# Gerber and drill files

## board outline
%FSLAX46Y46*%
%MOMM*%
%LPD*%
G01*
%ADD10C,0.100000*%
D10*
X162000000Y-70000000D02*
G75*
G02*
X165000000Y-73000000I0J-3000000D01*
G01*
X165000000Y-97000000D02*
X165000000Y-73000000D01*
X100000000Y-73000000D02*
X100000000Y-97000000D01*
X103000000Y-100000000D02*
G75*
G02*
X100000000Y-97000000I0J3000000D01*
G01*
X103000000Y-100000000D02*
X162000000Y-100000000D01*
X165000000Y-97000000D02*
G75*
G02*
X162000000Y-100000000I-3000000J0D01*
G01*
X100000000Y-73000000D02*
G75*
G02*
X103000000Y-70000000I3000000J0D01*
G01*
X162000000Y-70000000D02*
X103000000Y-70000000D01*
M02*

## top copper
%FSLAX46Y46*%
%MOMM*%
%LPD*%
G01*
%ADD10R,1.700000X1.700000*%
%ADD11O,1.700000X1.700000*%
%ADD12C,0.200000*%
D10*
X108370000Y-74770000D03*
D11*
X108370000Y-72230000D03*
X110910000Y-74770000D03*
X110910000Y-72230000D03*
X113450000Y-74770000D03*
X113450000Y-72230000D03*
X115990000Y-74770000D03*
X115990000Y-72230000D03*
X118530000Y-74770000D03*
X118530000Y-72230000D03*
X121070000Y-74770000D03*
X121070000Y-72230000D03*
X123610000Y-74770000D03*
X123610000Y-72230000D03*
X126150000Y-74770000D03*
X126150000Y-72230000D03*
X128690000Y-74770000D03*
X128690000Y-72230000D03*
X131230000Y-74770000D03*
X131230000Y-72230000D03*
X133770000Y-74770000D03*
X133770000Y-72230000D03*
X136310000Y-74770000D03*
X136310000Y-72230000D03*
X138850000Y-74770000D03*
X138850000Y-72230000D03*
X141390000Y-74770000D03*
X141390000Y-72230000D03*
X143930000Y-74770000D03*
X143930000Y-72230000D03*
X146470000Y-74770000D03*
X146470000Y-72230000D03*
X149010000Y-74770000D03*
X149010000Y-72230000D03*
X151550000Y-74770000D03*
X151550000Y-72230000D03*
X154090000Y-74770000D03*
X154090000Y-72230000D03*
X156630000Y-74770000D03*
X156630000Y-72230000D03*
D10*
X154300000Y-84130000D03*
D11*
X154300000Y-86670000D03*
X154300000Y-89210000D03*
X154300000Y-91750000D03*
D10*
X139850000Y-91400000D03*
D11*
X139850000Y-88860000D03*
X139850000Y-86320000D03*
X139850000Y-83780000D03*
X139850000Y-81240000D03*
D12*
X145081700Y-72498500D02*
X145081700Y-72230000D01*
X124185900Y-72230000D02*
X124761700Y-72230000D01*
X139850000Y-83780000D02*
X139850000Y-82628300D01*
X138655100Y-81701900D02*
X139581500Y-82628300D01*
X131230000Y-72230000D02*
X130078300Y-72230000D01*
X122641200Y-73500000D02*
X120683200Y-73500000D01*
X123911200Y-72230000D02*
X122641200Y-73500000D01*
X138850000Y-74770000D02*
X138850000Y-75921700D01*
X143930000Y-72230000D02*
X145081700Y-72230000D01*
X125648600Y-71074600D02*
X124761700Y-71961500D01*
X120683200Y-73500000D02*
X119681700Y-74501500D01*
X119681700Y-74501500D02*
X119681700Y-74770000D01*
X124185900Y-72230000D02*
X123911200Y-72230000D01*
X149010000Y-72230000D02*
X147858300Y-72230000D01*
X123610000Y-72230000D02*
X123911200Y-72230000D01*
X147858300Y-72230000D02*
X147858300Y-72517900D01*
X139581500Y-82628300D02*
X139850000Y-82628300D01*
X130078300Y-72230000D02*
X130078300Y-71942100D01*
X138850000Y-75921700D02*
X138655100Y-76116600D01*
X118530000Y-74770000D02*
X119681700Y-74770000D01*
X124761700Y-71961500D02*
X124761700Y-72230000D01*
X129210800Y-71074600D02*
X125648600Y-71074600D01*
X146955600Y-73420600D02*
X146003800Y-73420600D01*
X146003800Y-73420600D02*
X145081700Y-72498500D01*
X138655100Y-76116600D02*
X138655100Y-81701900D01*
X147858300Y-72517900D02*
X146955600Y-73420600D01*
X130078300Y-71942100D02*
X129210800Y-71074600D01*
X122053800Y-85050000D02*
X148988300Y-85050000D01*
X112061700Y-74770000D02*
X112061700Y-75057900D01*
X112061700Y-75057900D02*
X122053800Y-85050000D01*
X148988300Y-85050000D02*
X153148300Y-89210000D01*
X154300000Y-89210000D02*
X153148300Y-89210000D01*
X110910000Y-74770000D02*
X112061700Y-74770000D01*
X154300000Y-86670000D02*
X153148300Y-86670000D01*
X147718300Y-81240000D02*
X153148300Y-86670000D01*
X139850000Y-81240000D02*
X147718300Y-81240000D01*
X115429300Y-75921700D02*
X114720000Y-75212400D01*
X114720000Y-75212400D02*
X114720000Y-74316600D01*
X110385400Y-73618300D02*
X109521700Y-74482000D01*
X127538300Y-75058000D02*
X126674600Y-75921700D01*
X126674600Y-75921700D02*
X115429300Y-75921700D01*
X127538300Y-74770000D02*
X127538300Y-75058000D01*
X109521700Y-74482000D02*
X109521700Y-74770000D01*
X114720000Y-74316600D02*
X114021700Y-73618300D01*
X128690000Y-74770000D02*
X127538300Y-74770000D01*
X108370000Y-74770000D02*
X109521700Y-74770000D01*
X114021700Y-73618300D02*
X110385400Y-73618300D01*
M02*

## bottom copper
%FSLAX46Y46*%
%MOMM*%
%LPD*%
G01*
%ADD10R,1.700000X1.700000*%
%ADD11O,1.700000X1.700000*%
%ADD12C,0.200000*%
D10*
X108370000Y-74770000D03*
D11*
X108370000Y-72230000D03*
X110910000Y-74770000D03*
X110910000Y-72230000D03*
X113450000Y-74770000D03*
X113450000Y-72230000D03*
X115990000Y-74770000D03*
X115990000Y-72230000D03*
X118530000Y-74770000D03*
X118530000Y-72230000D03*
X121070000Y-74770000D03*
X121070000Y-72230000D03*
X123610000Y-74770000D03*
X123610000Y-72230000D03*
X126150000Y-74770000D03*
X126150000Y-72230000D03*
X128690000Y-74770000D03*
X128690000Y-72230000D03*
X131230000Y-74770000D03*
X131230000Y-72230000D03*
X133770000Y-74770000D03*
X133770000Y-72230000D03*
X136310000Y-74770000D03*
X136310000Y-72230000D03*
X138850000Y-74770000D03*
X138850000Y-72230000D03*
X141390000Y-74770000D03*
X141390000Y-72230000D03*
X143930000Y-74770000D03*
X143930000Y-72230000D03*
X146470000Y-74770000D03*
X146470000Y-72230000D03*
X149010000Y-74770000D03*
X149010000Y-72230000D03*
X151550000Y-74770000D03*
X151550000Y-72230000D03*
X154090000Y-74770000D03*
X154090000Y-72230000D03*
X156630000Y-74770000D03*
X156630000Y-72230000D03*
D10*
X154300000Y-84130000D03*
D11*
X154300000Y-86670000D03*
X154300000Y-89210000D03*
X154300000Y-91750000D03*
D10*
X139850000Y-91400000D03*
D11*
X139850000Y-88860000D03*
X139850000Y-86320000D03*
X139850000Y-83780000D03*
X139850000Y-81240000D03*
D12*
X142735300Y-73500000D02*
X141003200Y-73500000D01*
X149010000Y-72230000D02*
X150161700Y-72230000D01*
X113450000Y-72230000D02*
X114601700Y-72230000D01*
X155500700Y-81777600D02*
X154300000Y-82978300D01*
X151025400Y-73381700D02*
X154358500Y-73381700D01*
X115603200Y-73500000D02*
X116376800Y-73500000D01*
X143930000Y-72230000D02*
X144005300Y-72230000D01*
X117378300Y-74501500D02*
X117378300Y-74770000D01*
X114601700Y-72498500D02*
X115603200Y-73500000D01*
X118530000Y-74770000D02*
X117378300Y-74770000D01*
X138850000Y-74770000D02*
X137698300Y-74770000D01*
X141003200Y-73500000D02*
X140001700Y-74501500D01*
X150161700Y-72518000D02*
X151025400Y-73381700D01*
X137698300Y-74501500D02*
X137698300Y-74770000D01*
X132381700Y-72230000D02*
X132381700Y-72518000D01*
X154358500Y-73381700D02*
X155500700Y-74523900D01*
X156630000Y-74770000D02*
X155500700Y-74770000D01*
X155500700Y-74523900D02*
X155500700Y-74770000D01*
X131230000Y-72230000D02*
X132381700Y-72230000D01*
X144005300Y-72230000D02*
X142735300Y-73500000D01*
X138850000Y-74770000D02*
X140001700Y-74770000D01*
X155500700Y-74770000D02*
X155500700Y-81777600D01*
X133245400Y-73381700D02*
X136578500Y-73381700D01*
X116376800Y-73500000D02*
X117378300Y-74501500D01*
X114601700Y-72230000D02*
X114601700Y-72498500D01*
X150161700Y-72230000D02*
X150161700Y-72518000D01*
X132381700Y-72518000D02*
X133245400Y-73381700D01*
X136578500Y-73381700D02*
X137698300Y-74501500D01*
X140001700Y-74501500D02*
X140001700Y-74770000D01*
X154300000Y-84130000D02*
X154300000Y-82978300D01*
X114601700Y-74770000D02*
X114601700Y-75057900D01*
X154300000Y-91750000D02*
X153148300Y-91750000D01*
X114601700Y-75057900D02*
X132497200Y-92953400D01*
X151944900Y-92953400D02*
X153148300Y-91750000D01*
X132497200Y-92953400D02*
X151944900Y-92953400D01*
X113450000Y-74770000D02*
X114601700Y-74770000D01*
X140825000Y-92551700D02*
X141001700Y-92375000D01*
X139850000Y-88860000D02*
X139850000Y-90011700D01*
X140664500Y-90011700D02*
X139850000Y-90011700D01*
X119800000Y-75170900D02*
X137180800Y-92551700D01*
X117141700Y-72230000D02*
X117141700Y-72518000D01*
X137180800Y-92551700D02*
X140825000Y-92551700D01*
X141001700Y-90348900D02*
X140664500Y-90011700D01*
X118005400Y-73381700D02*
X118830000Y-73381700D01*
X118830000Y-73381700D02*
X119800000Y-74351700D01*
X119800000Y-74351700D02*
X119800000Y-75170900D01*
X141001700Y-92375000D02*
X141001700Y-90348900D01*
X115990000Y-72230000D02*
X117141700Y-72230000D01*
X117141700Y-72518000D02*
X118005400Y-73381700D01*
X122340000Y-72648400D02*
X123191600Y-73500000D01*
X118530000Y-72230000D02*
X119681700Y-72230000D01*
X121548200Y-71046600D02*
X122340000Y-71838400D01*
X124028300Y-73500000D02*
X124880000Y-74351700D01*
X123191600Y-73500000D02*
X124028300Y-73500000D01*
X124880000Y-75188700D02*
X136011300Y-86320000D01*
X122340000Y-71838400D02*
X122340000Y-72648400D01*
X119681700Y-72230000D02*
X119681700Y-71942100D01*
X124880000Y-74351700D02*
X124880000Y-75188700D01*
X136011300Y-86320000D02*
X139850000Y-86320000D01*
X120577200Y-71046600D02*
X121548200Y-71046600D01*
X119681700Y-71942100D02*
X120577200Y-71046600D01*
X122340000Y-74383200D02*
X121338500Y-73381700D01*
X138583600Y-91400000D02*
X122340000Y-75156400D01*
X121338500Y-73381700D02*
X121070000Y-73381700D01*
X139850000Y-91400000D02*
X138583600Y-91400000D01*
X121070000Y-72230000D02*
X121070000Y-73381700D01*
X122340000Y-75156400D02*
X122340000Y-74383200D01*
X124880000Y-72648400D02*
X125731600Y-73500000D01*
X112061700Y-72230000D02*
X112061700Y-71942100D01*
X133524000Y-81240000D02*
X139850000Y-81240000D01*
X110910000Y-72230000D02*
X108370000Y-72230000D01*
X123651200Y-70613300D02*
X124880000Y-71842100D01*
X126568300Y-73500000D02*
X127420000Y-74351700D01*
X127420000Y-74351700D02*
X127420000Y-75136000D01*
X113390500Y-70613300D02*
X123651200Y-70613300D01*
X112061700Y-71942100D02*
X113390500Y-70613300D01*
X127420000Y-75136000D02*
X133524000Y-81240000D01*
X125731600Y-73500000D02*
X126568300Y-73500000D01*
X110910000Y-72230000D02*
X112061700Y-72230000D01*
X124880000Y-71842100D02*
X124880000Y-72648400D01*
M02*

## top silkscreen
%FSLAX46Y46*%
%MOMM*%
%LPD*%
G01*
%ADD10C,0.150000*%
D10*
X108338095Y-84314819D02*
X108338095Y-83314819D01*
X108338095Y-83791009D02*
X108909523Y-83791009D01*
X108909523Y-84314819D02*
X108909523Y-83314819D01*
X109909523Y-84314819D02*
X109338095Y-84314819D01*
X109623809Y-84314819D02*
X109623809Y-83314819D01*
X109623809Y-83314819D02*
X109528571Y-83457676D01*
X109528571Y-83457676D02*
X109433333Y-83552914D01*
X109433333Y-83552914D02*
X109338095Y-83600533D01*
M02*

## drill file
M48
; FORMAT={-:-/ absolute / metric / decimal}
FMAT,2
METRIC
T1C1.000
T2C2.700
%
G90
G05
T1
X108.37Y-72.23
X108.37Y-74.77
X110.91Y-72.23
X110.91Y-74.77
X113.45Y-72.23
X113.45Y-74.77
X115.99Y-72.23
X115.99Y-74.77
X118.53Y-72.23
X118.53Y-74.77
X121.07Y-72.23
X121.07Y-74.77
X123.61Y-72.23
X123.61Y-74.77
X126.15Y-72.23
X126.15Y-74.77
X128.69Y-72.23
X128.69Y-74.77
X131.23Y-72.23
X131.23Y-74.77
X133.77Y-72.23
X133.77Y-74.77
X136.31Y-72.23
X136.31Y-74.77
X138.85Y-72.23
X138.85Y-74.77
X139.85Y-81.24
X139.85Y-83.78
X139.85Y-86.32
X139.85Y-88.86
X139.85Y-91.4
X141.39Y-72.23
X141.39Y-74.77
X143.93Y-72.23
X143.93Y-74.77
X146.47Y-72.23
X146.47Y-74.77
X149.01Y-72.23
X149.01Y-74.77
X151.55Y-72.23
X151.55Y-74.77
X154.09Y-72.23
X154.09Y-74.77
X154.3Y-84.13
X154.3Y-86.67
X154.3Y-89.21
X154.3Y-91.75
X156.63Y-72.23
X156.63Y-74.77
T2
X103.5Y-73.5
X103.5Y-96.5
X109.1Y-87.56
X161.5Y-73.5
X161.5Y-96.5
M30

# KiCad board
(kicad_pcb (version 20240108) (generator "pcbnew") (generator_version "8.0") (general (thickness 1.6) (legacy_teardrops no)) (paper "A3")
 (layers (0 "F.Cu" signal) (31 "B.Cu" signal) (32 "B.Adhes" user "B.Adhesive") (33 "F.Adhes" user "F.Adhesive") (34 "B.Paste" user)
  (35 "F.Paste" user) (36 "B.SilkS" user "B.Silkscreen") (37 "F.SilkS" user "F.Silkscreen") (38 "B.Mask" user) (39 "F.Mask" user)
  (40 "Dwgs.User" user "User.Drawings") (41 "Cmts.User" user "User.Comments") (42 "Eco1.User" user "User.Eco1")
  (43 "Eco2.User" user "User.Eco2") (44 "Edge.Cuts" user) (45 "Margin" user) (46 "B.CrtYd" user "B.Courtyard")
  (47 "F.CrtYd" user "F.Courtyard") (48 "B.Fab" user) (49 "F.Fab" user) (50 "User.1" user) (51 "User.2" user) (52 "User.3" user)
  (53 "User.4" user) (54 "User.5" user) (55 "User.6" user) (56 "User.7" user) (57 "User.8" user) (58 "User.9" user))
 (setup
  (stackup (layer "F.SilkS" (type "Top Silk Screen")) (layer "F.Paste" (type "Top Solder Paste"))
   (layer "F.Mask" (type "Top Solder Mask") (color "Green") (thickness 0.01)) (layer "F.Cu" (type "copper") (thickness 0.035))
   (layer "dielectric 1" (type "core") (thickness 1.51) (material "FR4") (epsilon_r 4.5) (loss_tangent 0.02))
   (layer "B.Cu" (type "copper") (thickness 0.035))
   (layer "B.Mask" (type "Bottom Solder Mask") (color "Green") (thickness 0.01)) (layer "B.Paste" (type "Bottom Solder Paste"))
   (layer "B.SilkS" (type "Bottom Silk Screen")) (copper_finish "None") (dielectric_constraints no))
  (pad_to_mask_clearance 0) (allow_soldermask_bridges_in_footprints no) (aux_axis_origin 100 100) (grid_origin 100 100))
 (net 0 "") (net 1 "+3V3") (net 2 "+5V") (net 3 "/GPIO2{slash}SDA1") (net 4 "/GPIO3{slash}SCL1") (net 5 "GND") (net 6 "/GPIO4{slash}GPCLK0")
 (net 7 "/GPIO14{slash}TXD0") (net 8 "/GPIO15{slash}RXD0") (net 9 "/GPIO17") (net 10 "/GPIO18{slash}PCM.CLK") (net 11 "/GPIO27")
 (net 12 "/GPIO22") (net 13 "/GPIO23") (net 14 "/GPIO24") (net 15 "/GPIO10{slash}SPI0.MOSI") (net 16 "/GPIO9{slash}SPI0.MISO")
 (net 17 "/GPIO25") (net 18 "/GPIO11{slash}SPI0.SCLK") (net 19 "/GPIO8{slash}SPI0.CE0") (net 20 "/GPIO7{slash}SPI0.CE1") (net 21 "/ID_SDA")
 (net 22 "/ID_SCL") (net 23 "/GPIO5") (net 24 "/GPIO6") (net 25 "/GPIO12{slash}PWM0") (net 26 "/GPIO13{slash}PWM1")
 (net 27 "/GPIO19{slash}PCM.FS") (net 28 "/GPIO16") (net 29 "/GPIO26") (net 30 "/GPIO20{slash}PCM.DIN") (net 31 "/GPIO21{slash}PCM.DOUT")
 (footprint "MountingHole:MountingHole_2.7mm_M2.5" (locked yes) (layer "F.Cu") (at 161.5 73.5)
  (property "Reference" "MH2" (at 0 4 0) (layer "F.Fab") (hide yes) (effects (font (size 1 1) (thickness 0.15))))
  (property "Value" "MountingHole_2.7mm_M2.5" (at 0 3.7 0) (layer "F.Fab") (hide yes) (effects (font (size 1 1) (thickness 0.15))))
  (pad "" np_thru_hole circle (at 0 0) (size 2.7 2.7) (drill 2.7) (layers "*.Cu" "*.Mask")))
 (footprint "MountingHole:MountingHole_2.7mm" (layer "F.Cu") (at 109.1 87.56)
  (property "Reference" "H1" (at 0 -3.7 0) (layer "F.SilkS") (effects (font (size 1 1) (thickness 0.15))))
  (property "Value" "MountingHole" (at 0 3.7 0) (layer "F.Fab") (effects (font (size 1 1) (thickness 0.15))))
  (pad "" np_thru_hole circle (at 0 0) (size 2.7 2.7) (drill 2.7) (layers "*.Cu" "*.Mask")))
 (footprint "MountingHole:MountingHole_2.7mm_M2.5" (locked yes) (layer "F.Cu") (at 103.5 96.5)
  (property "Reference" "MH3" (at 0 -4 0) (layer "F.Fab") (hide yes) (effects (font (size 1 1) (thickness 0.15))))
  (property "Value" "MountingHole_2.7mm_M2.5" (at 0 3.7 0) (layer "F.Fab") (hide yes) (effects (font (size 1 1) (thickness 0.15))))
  (pad "" np_thru_hole circle (at 0 0) (size 2.7 2.7) (drill 2.7) (layers "*.Cu" "*.Mask")))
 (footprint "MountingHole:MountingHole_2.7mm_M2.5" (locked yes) (layer "F.Cu") (at 103.5 73.5)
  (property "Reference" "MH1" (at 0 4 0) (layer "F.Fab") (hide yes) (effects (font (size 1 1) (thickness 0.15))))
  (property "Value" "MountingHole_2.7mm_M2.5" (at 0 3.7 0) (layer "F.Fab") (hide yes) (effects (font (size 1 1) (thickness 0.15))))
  (pad "" np_thru_hole circle (at 0 0) (size 2.7 2.7) (drill 2.7) (layers "*.Cu" "*.Mask")))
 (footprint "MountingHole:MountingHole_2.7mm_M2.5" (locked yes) (layer "F.Cu") (at 161.5 96.5)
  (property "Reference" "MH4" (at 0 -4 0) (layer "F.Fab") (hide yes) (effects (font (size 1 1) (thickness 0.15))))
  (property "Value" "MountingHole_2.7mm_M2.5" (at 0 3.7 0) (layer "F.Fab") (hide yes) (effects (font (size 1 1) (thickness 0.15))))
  (pad "" np_thru_hole circle (at 0 0) (size 2.7 2.7) (drill 2.7) (layers "*.Cu" "*.Mask")))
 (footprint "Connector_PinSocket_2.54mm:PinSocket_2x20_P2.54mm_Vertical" (layer "B.Cu") (at 108.37 74.77 -90)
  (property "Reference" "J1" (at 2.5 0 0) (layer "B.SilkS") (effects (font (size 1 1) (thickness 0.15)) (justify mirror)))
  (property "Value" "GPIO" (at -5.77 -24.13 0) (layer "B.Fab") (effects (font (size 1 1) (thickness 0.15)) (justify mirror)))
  (pad "1" thru_hole rect (at 0 0 270) (size 1.7 1.7) (drill 1) (layers "*.Cu" "*.Mask") (remove_unused_layers no) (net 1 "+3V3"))
  (pad "2" thru_hole oval (at -2.54 0 270) (size 1.7 1.7) (drill 1) (layers "*.Cu" "*.Mask") (remove_unused_layers no) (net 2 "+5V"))
  (pad "3" thru_hole oval (at 0 -2.54 270) (size 1.7 1.7) (drill 1) (layers "*.Cu" "*.Mask") (remove_unused_layers no)
   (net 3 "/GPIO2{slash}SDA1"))
  (pad "4" thru_hole oval (at -2.54 -2.54 270) (size 1.7 1.7) (drill 1) (layers "*.Cu" "*.Mask") (remove_unused_layers no) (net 2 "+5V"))
  (pad "5" thru_hole oval (at 0 -5.08 270) (size 1.7 1.7) (drill 1) (layers "*.Cu" "*.Mask") (remove_unused_layers no)
   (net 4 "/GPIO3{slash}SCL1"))
  (pad "6" thru_hole oval (at -2.54 -5.08 270) (size 1.7 1.7) (drill 1) (layers "*.Cu" "*.Mask") (remove_unused_layers no) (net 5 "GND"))
  (pad "7" thru_hole oval (at 0 -7.62 270) (size 1.7 1.7) (drill 1) (layers "*.Cu" "*.Mask") (remove_unused_layers no)
   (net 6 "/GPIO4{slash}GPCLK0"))
  (pad "8" thru_hole oval (at -2.54 -7.62 270) (size 1.7 1.7) (drill 1) (layers "*.Cu" "*.Mask") (remove_unused_layers no)
   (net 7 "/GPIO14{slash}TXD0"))
  (pad "9" thru_hole oval (at 0 -10.16 270) (size 1.7 1.7) (drill 1) (layers "*.Cu" "*.Mask") (remove_unused_layers no) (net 5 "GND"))
  (pad "10" thru_hole oval (at -2.54 -10.16 270) (size 1.7 1.7) (drill 1) (layers "*.Cu" "*.Mask") (remove_unused_layers no)
   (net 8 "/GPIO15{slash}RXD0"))
  (pad "11" thru_hole oval (at 0 -12.7 270) (size 1.7 1.7) (drill 1) (layers "*.Cu" "*.Mask") (remove_unused_layers no) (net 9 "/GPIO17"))
  (pad "12" thru_hole oval (at -2.54 -12.7 270) (size 1.7 1.7) (drill 1) (layers "*.Cu" "*.Mask") (remove_unused_layers no)
   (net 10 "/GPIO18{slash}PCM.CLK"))
  (pad "13" thru_hole oval (at 0 -15.24 270) (size 1.7 1.7) (drill 1) (layers "*.Cu" "*.Mask") (remove_unused_layers no) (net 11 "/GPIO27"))
  (pad "14" thru_hole oval (at -2.54 -15.24 270) (size 1.7 1.7) (drill 1) (layers "*.Cu" "*.Mask") (remove_unused_layers no) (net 5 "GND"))
  (pad "15" thru_hole oval (at 0 -17.78 270) (size 1.7 1.7) (drill 1) (layers "*.Cu" "*.Mask") (remove_unused_layers no) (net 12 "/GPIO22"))
  (pad "16" thru_hole oval (at -2.54 -17.78 270) (size 1.7 1.7) (drill 1) (layers "*.Cu" "*.Mask") (remove_unused_layers no)
   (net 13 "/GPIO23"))
  (pad "17" thru_hole oval (at 0 -20.32 270) (size 1.7 1.7) (drill 1) (layers "*.Cu" "*.Mask") (remove_unused_layers no) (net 1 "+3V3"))
  (pad "18" thru_hole oval (at -2.54 -20.32 270) (size 1.7 1.7) (drill 1) (layers "*.Cu" "*.Mask") (remove_unused_layers no)
   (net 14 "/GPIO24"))
  (pad "19" thru_hole oval (at 0 -22.86 270) (size 1.7 1.7) (drill 1) (layers "*.Cu" "*.Mask") (remove_unused_layers no)
   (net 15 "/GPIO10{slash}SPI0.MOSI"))
  (pad "20" thru_hole oval (at -2.54 -22.86 270) (size 1.7 1.7) (drill 1) (layers "*.Cu" "*.Mask") (remove_unused_layers no) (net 5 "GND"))
  (pad "21" thru_hole oval (at 0 -25.4 270) (size 1.7 1.7) (drill 1) (layers "*.Cu" "*.Mask") (remove_unused_layers no)
   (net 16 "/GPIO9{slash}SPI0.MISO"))
  (pad "22" thru_hole oval (at -2.54 -25.4 270) (size 1.7 1.7) (drill 1) (layers "*.Cu" "*.Mask") (remove_unused_layers no)
   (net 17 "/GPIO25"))
  (pad "23" thru_hole oval (at 0 -27.94 270) (size 1.7 1.7) (drill 1) (layers "*.Cu" "*.Mask") (remove_unused_layers no)
   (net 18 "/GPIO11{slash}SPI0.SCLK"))
  (pad "24" thru_hole oval (at -2.54 -27.94 270) (size 1.7 1.7) (drill 1) (layers "*.Cu" "*.Mask") (remove_unused_layers no)
   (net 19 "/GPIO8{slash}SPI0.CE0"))
  (pad "25" thru_hole oval (at 0 -30.48 270) (size 1.7 1.7) (drill 1) (layers "*.Cu" "*.Mask") (remove_unused_layers no) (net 5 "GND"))
  (pad "26" thru_hole oval (at -2.54 -30.48 270) (size 1.7 1.7) (drill 1) (layers "*.Cu" "*.Mask") (remove_unused_layers no)
   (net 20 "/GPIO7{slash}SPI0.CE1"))
  (pad "27" thru_hole oval (at 0 -33.02 270) (size 1.7 1.7) (drill 1) (layers "*.Cu" "*.Mask") (remove_unused_layers no) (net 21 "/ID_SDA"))
  (pad "28" thru_hole oval (at -2.54 -33.02 270) (size 1.7 1.7) (drill 1) (layers "*.Cu" "*.Mask") (remove_unused_layers no)
   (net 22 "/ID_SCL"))
  (pad "29" thru_hole oval (at 0 -35.56 270) (size 1.7 1.7) (drill 1) (layers "*.Cu" "*.Mask") (remove_unused_layers no) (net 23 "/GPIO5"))
  (pad "30" thru_hole oval (at -2.54 -35.56 270) (size 1.7 1.7) (drill 1) (layers "*.Cu" "*.Mask") (remove_unused_layers no) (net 5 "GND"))
  (pad "31" thru_hole oval (at 0 -38.1 270) (size 1.7 1.7) (drill 1) (layers "*.Cu" "*.Mask") (remove_unused_layers no) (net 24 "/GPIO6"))
  (pad "32" thru_hole oval (at -2.54 -38.1 270) (size 1.7 1.7) (drill 1) (layers "*.Cu" "*.Mask") (remove_unused_layers no)
   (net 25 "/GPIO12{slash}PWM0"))
  (pad "33" thru_hole oval (at 0 -40.64 270) (size 1.7 1.7) (drill 1) (layers "*.Cu" "*.Mask") (remove_unused_layers no)
   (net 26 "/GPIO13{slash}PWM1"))
  (pad "34" thru_hole oval (at -2.54 -40.64 270) (size 1.7 1.7) (drill 1) (layers "*.Cu" "*.Mask") (remove_unused_layers no) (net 5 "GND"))
  (pad "35" thru_hole oval (at 0 -43.18 270) (size 1.7 1.7) (drill 1) (layers "*.Cu" "*.Mask") (remove_unused_layers no)
   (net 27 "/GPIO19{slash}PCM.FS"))
  (pad "36" thru_hole oval (at -2.54 -43.18 270) (size 1.7 1.7) (drill 1) (layers "*.Cu" "*.Mask") (remove_unused_layers no)
   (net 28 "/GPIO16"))
  (pad "37" thru_hole oval (at 0 -45.72 270) (size 1.7 1.7) (drill 1) (layers "*.Cu" "*.Mask") (remove_unused_layers no) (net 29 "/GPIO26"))
  (pad "38" thru_hole oval (at -2.54 -45.72 270) (size 1.7 1.7) (drill 1) (layers "*.Cu" "*.Mask") (remove_unused_layers no)
   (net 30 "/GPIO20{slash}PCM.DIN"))
  (pad "39" thru_hole oval (at 0 -48.26 270) (size 1.7 1.7) (drill 1) (layers "*.Cu" "*.Mask") (remove_unused_layers no) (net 5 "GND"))
  (pad "40" thru_hole oval (at -2.54 -48.26 270) (size 1.7 1.7) (drill 1) (layers "*.Cu" "*.Mask") (remove_unused_layers no)
   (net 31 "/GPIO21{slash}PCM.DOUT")))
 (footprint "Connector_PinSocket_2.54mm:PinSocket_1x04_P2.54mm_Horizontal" (layer "B.Cu") (at 154.3 84.13 180)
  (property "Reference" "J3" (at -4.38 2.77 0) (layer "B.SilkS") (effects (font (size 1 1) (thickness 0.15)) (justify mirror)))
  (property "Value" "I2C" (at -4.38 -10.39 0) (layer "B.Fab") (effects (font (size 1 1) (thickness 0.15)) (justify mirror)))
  (pad "1" thru_hole rect (at 0 0 180) (size 1.7 1.7) (drill 1) (layers "*.Cu" "*.Mask") (remove_unused_layers no) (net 5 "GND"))
  (pad "2" thru_hole oval (at 0 -2.54 180) (size 1.7 1.7) (drill 1) (layers "*.Cu" "*.Mask") (remove_unused_layers no) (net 2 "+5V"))
  (pad "3" thru_hole oval (at 0 -5.08 180) (size 1.7 1.7) (drill 1) (layers "*.Cu" "*.Mask") (remove_unused_layers no)
   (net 3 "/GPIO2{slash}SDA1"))
  (pad "4" thru_hole oval (at 0 -7.62 180) (size 1.7 1.7) (drill 1) (layers "*.Cu" "*.Mask") (remove_unused_layers no)
   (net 4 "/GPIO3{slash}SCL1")))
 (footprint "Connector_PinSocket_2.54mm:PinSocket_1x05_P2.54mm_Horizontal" (layer "B.Cu") (at 139.85 91.4)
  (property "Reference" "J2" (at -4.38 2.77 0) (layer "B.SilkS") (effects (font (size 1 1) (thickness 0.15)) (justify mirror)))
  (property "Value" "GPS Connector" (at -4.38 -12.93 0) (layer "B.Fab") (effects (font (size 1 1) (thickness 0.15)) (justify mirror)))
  (pad "1" thru_hole rect (at 0 0) (size 1.7 1.7) (drill 1) (layers "*.Cu" "*.Mask") (remove_unused_layers no)
   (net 10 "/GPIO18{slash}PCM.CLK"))
  (pad "2" thru_hole oval (at 0 -2.54) (size 1.7 1.7) (drill 1) (layers "*.Cu" "*.Mask") (remove_unused_layers no)
   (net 7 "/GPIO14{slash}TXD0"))
  (pad "3" thru_hole oval (at 0 -5.08) (size 1.7 1.7) (drill 1) (layers "*.Cu" "*.Mask") (remove_unused_layers no)
   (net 8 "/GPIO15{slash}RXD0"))
  (pad "4" thru_hole oval (at 0 -7.62) (size 1.7 1.7) (drill 1) (layers "*.Cu" "*.Mask") (remove_unused_layers no) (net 5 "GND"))
  (pad "5" thru_hole oval (at 0 -10.16) (size 1.7 1.7) (drill 1) (layers "*.Cu" "*.Mask") (remove_unused_layers no) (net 2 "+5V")))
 (gr_arc (start 162 70) (mid 164.12132 70.87868) (end 165 73) (stroke (width 0.1) (type solid)) (layer "Edge.Cuts"))
 (gr_line (start 165 97) (end 165 73) (stroke (width 0.1) (type solid)) (layer "Edge.Cuts"))
 (gr_line (start 100 73) (end 100 97) (stroke (width 0.1) (type solid)) (layer "Edge.Cuts"))
 (gr_arc (start 103 100) (mid 100.87868 99.12132) (end 100 97) (stroke (width 0.1) (type solid)) (layer "Edge.Cuts"))
 (gr_line (start 103 100) (end 162 100) (stroke (width 0.1) (type solid)) (layer "Edge.Cuts"))
 (gr_arc (start 165 97) (mid 164.12132 99.12132) (end 162 100) (stroke (width 0.1) (type solid)) (layer "Edge.Cuts"))
 (gr_arc (start 100 73) (mid 100.87868 70.87868) (end 103 70) (stroke (width 0.1) (type solid)) (layer "Edge.Cuts"))
 (gr_line (start 162 70) (end 103 70) (stroke (width 0.1) (type solid)) (layer "Edge.Cuts"))
 (segment (start 145.0817 72.4985) (end 145.0817 72.23) (width 0.2) (layer "F.Cu") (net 5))
 (segment (start 124.1859 72.23) (end 124.7617 72.23) (width 0.2) (layer "F.Cu") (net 5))
 (segment (start 139.85 83.78) (end 139.85 82.6283) (width 0.2) (layer "F.Cu") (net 5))
 (segment (start 138.6551 81.7019) (end 139.5815 82.6283) (width 0.2) (layer "F.Cu") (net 5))
 (segment (start 131.23 72.23) (end 130.0783 72.23) (width 0.2) (layer "F.Cu") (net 5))
 (segment (start 122.6412 73.5) (end 120.6832 73.5) (width 0.2) (layer "F.Cu") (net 5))
 (segment (start 123.9112 72.23) (end 122.6412 73.5) (width 0.2) (layer "F.Cu") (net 5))
 (segment (start 138.85 74.77) (end 138.85 75.9217) (width 0.2) (layer "F.Cu") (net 5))
 (segment (start 143.93 72.23) (end 145.0817 72.23) (width 0.2) (layer "F.Cu") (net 5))
 (segment (start 125.6486 71.0746) (end 124.7617 71.9615) (width 0.2) (layer "F.Cu") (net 5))
 (segment (start 120.6832 73.5) (end 119.6817 74.5015) (width 0.2) (layer "F.Cu") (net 5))
 (segment (start 119.6817 74.5015) (end 119.6817 74.77) (width 0.2) (layer "F.Cu") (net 5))
 (segment (start 124.1859 72.23) (end 123.9112 72.23) (width 0.2) (layer "F.Cu") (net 5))
 (segment (start 149.01 72.23) (end 147.8583 72.23) (width 0.2) (layer "F.Cu") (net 5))
 (segment (start 123.61 72.23) (end 123.9112 72.23) (width 0.2) (layer "F.Cu") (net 5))
 (segment (start 147.8583 72.23) (end 147.8583 72.5179) (width 0.2) (layer "F.Cu") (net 5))
 (segment (start 139.5815 82.6283) (end 139.85 82.6283) (width 0.2) (layer "F.Cu") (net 5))
 (segment (start 130.0783 72.23) (end 130.0783 71.9421) (width 0.2) (layer "F.Cu") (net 5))
 (segment (start 138.85 75.9217) (end 138.6551 76.1166) (width 0.2) (layer "F.Cu") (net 5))
 (segment (start 118.53 74.77) (end 119.6817 74.77) (width 0.2) (layer "F.Cu") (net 5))
 (segment (start 124.7617 71.9615) (end 124.7617 72.23) (width 0.2) (layer "F.Cu") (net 5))
 (segment (start 129.2108 71.0746) (end 125.6486 71.0746) (width 0.2) (layer "F.Cu") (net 5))
 (segment (start 146.9556 73.4206) (end 146.0038 73.4206) (width 0.2) (layer "F.Cu") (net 5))
 (segment (start 146.0038 73.4206) (end 145.0817 72.4985) (width 0.2) (layer "F.Cu") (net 5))
 (segment (start 138.6551 76.1166) (end 138.6551 81.7019) (width 0.2) (layer "F.Cu") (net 5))
 (segment (start 147.8583 72.5179) (end 146.9556 73.4206) (width 0.2) (layer "F.Cu") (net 5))
 (segment (start 130.0783 71.9421) (end 129.2108 71.0746) (width 0.2) (layer "F.Cu") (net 5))
 (segment (start 142.7353 73.5) (end 141.0032 73.5) (width 0.2) (layer "B.Cu") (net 5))
 (segment (start 149.01 72.23) (end 150.1617 72.23) (width 0.2) (layer "B.Cu") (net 5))
 (segment (start 113.45 72.23) (end 114.6017 72.23) (width 0.2) (layer "B.Cu") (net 5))
 (segment (start 155.5007 81.7776) (end 154.3 82.9783) (width 0.2) (layer "B.Cu") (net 5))
 (segment (start 151.0254 73.3817) (end 154.3585 73.3817) (width 0.2) (layer "B.Cu") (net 5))
 (segment (start 115.6032 73.5) (end 116.3768 73.5) (width 0.2) (layer "B.Cu") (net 5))
 (segment (start 143.93 72.23) (end 144.0053 72.23) (width 0.2) (layer "B.Cu") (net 5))
 (segment (start 117.3783 74.5015) (end 117.3783 74.77) (width 0.2) (layer "B.Cu") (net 5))
 (segment (start 114.6017 72.4985) (end 115.6032 73.5) (width 0.2) (layer "B.Cu") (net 5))
 (segment (start 118.53 74.77) (end 117.3783 74.77) (width 0.2) (layer "B.Cu") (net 5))
 (segment (start 138.85 74.77) (end 137.6983 74.77) (width 0.2) (layer "B.Cu") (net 5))
 (segment (start 141.0032 73.5) (end 140.0017 74.5015) (width 0.2) (layer "B.Cu") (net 5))
 (segment (start 150.1617 72.518) (end 151.0254 73.3817) (width 0.2) (layer "B.Cu") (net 5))
 (segment (start 137.6983 74.5015) (end 137.6983 74.77) (width 0.2) (layer "B.Cu") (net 5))
 (segment (start 132.3817 72.23) (end 132.3817 72.518) (width 0.2) (layer "B.Cu") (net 5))
 (segment (start 154.3585 73.3817) (end 155.5007 74.5239) (width 0.2) (layer "B.Cu") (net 5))
 (segment (start 156.63 74.77) (end 155.5007 74.77) (width 0.2) (layer "B.Cu") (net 5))
 (segment (start 155.5007 74.5239) (end 155.5007 74.77) (width 0.2) (layer "B.Cu") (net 5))
 (segment (start 131.23 72.23) (end 132.3817 72.23) (width 0.2) (layer "B.Cu") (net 5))
 (segment (start 144.0053 72.23) (end 142.7353 73.5) (width 0.2) (layer "B.Cu") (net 5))
 (segment (start 138.85 74.77) (end 140.0017 74.77) (width 0.2) (layer "B.Cu") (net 5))
 (segment (start 155.5007 74.77) (end 155.5007 81.7776) (width 0.2) (layer "B.Cu") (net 5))
 (segment (start 133.2454 73.3817) (end 136.5785 73.3817) (width 0.2) (layer "B.Cu") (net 5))
 (segment (start 116.3768 73.5) (end 117.3783 74.5015) (width 0.2) (layer "B.Cu") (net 5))
 (segment (start 114.6017 72.23) (end 114.6017 72.4985) (width 0.2) (layer "B.Cu") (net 5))
 (segment (start 150.1617 72.23) (end 150.1617 72.518) (width 0.2) (layer "B.Cu") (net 5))
 (segment (start 132.3817 72.518) (end 133.2454 73.3817) (width 0.2) (layer "B.Cu") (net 5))
 (segment (start 136.5785 73.3817) (end 137.6983 74.5015) (width 0.2) (layer "B.Cu") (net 5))
 (segment (start 140.0017 74.5015) (end 140.0017 74.77) (width 0.2) (layer "B.Cu") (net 5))
 (segment (start 154.3 84.13) (end 154.3 82.9783) (width 0.2) (layer "B.Cu") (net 5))
 (segment (start 122.0538 85.05) (end 148.9883 85.05) (width 0.2) (layer "F.Cu") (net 3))
 (segment (start 112.0617 74.77) (end 112.0617 75.0579) (width 0.2) (layer "F.Cu") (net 3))
 (segment (start 112.0617 75.0579) (end 122.0538 85.05) (width 0.2) (layer "F.Cu") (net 3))
 (segment (start 148.9883 85.05) (end 153.1483 89.21) (width 0.2) (layer "F.Cu") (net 3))
 (segment (start 154.3 89.21) (end 153.1483 89.21) (width 0.2) (layer "F.Cu") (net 3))
 (segment (start 110.91 74.77) (end 112.0617 74.77) (width 0.2) (layer "F.Cu") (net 3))
 (segment (start 114.6017 74.77) (end 114.6017 75.0579) (width 0.2) (layer "B.Cu") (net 4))
 (segment (start 154.3 91.75) (end 153.1483 91.75) (width 0.2) (layer "B.Cu") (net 4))
 (segment (start 114.6017 75.0579) (end 132.4972 92.9534) (width 0.2) (layer "B.Cu") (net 4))
 (segment (start 151.9449 92.9534) (end 153.1483 91.75) (width 0.2) (layer "B.Cu") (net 4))
 (segment (start 132.4972 92.9534) (end 151.9449 92.9534) (width 0.2) (layer "B.Cu") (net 4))
 (segment (start 113.45 74.77) (end 114.6017 74.77) (width 0.2) (layer "B.Cu") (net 4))
 (segment (start 140.825 92.5517) (end 141.0017 92.375) (width 0.2) (layer "B.Cu") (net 7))
 (segment (start 139.85 88.86) (end 139.85 90.0117) (width 0.2) (layer "B.Cu") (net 7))
 (segment (start 140.6645 90.0117) (end 139.85 90.0117) (width 0.2) (layer "B.Cu") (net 7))
 (segment (start 119.8 75.1709) (end 137.1808 92.5517) (width 0.2) (layer "B.Cu") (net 7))
 (segment (start 117.1417 72.23) (end 117.1417 72.518) (width 0.2) (layer "B.Cu") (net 7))
 (segment (start 137.1808 92.5517) (end 140.825 92.5517) (width 0.2) (layer "B.Cu") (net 7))
 (segment (start 141.0017 90.3489) (end 140.6645 90.0117) (width 0.2) (layer "B.Cu") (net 7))
 (segment (start 118.0054 73.3817) (end 118.83 73.3817) (width 0.2) (layer "B.Cu") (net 7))
 (segment (start 118.83 73.3817) (end 119.8 74.3517) (width 0.2) (layer "B.Cu") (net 7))
 (segment (start 119.8 74.3517) (end 119.8 75.1709) (width 0.2) (layer "B.Cu") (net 7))
 (segment (start 141.0017 92.375) (end 141.0017 90.3489) (width 0.2) (layer "B.Cu") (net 7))
 (segment (start 115.99 72.23) (end 117.1417 72.23) (width 0.2) (layer "B.Cu") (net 7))
 (segment (start 117.1417 72.518) (end 118.0054 73.3817) (width 0.2) (layer "B.Cu") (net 7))
 (segment (start 122.34 72.6484) (end 123.1916 73.5) (width 0.2) (layer "B.Cu") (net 8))
 (segment (start 118.53 72.23) (end 119.6817 72.23) (width 0.2) (layer "B.Cu") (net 8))
 (segment (start 121.5482 71.0466) (end 122.34 71.8384) (width 0.2) (layer "B.Cu") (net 8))
 (segment (start 124.0283 73.5) (end 124.88 74.3517) (width 0.2) (layer "B.Cu") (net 8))
 (segment (start 123.1916 73.5) (end 124.0283 73.5) (width 0.2) (layer "B.Cu") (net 8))
 (segment (start 124.88 75.1887) (end 136.0113 86.32) (width 0.2) (layer "B.Cu") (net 8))
 (segment (start 122.34 71.8384) (end 122.34 72.6484) (width 0.2) (layer "B.Cu") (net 8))
 (segment (start 119.6817 72.23) (end 119.6817 71.9421) (width 0.2) (layer "B.Cu") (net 8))
 (segment (start 124.88 74.3517) (end 124.88 75.1887) (width 0.2) (layer "B.Cu") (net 8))
 (segment (start 136.0113 86.32) (end 139.85 86.32) (width 0.2) (layer "B.Cu") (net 8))
 (segment (start 120.5772 71.0466) (end 121.5482 71.0466) (width 0.2) (layer "B.Cu") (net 8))
 (segment (start 119.6817 71.9421) (end 120.5772 71.0466) (width 0.2) (layer "B.Cu") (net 8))
 (segment (start 122.34 74.3832) (end 121.3385 73.3817) (width 0.2) (layer "B.Cu") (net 10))
 (segment (start 138.5836 91.4) (end 122.34 75.1564) (width 0.2) (layer "B.Cu") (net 10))
 (segment (start 121.3385 73.3817) (end 121.07 73.3817) (width 0.2) (layer "B.Cu") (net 10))
 (segment (start 139.85 91.4) (end 138.5836 91.4) (width 0.2) (layer "B.Cu") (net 10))
 (segment (start 121.07 72.23) (end 121.07 73.3817) (width 0.2) (layer "B.Cu") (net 10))
 (segment (start 122.34 75.1564) (end 122.34 74.3832) (width 0.2) (layer "B.Cu") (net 10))
 (segment (start 154.3 86.67) (end 153.1483 86.67) (width 0.2) (layer "F.Cu") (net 2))
 (segment (start 147.7183 81.24) (end 153.1483 86.67) (width 0.2) (layer "F.Cu") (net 2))
 (segment (start 139.85 81.24) (end 147.7183 81.24) (width 0.2) (layer "F.Cu") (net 2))
 (segment (start 124.88 72.6484) (end 125.7316 73.5) (width 0.2) (layer "B.Cu") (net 2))
 (segment (start 112.0617 72.23) (end 112.0617 71.9421) (width 0.2) (layer "B.Cu") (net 2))
 (segment (start 133.524 81.24) (end 139.85 81.24) (width 0.2) (layer "B.Cu") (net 2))
 (segment (start 110.91 72.23) (end 108.37 72.23) (width 0.2) (layer "B.Cu") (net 2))
 (segment (start 123.6512 70.6133) (end 124.88 71.8421) (width 0.2) (layer "B.Cu") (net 2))
 (segment (start 126.5683 73.5) (end 127.42 74.3517) (width 0.2) (layer "B.Cu") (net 2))
 (segment (start 127.42 74.3517) (end 127.42 75.136) (width 0.2) (layer "B.Cu") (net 2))
 (segment (start 113.3905 70.6133) (end 123.6512 70.6133) (width 0.2) (layer "B.Cu") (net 2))
 (segment (start 112.0617 71.9421) (end 113.3905 70.6133) (width 0.2) (layer "B.Cu") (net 2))
 (segment (start 127.42 75.136) (end 133.524 81.24) (width 0.2) (layer "B.Cu") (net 2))
 (segment (start 125.7316 73.5) (end 126.5683 73.5) (width 0.2) (layer "B.Cu") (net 2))
 (segment (start 110.91 72.23) (end 112.0617 72.23) (width 0.2) (layer "B.Cu") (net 2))
 (segment (start 124.88 71.8421) (end 124.88 72.6484) (width 0.2) (layer "B.Cu") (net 2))
 (segment (start 115.4293 75.9217) (end 114.72 75.2124) (width 0.2) (layer "F.Cu") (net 1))
 (segment (start 114.72 75.2124) (end 114.72 74.3166) (width 0.2) (layer "F.Cu") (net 1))
 (segment (start 110.3854 73.6183) (end 109.5217 74.482) (width 0.2) (layer "F.Cu") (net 1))
 (segment (start 127.5383 75.058) (end 126.6746 75.9217) (width 0.2) (layer "F.Cu") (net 1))
 (segment (start 126.6746 75.9217) (end 115.4293 75.9217) (width 0.2) (layer "F.Cu") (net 1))
 (segment (start 127.5383 74.77) (end 127.5383 75.058) (width 0.2) (layer "F.Cu") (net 1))
 (segment (start 109.5217 74.482) (end 109.5217 74.77) (width 0.2) (layer "F.Cu") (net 1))
 (segment (start 114.72 74.3166) (end 114.0217 73.6183) (width 0.2) (layer "F.Cu") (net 1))
 (segment (start 128.69 74.77) (end 127.5383 74.77) (width 0.2) (layer "F.Cu") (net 1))
 (segment (start 108.37 74.77) (end 109.5217 74.77) (width 0.2) (layer "F.Cu") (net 1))
 (segment (start 114.0217 73.6183) (end 110.3854 73.6183) (width 0.2) (layer "F.Cu") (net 1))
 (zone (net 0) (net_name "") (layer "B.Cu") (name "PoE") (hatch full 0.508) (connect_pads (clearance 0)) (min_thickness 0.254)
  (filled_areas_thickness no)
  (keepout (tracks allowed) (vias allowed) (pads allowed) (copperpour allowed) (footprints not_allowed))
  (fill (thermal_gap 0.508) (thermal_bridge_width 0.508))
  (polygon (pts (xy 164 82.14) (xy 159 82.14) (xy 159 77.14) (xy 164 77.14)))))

